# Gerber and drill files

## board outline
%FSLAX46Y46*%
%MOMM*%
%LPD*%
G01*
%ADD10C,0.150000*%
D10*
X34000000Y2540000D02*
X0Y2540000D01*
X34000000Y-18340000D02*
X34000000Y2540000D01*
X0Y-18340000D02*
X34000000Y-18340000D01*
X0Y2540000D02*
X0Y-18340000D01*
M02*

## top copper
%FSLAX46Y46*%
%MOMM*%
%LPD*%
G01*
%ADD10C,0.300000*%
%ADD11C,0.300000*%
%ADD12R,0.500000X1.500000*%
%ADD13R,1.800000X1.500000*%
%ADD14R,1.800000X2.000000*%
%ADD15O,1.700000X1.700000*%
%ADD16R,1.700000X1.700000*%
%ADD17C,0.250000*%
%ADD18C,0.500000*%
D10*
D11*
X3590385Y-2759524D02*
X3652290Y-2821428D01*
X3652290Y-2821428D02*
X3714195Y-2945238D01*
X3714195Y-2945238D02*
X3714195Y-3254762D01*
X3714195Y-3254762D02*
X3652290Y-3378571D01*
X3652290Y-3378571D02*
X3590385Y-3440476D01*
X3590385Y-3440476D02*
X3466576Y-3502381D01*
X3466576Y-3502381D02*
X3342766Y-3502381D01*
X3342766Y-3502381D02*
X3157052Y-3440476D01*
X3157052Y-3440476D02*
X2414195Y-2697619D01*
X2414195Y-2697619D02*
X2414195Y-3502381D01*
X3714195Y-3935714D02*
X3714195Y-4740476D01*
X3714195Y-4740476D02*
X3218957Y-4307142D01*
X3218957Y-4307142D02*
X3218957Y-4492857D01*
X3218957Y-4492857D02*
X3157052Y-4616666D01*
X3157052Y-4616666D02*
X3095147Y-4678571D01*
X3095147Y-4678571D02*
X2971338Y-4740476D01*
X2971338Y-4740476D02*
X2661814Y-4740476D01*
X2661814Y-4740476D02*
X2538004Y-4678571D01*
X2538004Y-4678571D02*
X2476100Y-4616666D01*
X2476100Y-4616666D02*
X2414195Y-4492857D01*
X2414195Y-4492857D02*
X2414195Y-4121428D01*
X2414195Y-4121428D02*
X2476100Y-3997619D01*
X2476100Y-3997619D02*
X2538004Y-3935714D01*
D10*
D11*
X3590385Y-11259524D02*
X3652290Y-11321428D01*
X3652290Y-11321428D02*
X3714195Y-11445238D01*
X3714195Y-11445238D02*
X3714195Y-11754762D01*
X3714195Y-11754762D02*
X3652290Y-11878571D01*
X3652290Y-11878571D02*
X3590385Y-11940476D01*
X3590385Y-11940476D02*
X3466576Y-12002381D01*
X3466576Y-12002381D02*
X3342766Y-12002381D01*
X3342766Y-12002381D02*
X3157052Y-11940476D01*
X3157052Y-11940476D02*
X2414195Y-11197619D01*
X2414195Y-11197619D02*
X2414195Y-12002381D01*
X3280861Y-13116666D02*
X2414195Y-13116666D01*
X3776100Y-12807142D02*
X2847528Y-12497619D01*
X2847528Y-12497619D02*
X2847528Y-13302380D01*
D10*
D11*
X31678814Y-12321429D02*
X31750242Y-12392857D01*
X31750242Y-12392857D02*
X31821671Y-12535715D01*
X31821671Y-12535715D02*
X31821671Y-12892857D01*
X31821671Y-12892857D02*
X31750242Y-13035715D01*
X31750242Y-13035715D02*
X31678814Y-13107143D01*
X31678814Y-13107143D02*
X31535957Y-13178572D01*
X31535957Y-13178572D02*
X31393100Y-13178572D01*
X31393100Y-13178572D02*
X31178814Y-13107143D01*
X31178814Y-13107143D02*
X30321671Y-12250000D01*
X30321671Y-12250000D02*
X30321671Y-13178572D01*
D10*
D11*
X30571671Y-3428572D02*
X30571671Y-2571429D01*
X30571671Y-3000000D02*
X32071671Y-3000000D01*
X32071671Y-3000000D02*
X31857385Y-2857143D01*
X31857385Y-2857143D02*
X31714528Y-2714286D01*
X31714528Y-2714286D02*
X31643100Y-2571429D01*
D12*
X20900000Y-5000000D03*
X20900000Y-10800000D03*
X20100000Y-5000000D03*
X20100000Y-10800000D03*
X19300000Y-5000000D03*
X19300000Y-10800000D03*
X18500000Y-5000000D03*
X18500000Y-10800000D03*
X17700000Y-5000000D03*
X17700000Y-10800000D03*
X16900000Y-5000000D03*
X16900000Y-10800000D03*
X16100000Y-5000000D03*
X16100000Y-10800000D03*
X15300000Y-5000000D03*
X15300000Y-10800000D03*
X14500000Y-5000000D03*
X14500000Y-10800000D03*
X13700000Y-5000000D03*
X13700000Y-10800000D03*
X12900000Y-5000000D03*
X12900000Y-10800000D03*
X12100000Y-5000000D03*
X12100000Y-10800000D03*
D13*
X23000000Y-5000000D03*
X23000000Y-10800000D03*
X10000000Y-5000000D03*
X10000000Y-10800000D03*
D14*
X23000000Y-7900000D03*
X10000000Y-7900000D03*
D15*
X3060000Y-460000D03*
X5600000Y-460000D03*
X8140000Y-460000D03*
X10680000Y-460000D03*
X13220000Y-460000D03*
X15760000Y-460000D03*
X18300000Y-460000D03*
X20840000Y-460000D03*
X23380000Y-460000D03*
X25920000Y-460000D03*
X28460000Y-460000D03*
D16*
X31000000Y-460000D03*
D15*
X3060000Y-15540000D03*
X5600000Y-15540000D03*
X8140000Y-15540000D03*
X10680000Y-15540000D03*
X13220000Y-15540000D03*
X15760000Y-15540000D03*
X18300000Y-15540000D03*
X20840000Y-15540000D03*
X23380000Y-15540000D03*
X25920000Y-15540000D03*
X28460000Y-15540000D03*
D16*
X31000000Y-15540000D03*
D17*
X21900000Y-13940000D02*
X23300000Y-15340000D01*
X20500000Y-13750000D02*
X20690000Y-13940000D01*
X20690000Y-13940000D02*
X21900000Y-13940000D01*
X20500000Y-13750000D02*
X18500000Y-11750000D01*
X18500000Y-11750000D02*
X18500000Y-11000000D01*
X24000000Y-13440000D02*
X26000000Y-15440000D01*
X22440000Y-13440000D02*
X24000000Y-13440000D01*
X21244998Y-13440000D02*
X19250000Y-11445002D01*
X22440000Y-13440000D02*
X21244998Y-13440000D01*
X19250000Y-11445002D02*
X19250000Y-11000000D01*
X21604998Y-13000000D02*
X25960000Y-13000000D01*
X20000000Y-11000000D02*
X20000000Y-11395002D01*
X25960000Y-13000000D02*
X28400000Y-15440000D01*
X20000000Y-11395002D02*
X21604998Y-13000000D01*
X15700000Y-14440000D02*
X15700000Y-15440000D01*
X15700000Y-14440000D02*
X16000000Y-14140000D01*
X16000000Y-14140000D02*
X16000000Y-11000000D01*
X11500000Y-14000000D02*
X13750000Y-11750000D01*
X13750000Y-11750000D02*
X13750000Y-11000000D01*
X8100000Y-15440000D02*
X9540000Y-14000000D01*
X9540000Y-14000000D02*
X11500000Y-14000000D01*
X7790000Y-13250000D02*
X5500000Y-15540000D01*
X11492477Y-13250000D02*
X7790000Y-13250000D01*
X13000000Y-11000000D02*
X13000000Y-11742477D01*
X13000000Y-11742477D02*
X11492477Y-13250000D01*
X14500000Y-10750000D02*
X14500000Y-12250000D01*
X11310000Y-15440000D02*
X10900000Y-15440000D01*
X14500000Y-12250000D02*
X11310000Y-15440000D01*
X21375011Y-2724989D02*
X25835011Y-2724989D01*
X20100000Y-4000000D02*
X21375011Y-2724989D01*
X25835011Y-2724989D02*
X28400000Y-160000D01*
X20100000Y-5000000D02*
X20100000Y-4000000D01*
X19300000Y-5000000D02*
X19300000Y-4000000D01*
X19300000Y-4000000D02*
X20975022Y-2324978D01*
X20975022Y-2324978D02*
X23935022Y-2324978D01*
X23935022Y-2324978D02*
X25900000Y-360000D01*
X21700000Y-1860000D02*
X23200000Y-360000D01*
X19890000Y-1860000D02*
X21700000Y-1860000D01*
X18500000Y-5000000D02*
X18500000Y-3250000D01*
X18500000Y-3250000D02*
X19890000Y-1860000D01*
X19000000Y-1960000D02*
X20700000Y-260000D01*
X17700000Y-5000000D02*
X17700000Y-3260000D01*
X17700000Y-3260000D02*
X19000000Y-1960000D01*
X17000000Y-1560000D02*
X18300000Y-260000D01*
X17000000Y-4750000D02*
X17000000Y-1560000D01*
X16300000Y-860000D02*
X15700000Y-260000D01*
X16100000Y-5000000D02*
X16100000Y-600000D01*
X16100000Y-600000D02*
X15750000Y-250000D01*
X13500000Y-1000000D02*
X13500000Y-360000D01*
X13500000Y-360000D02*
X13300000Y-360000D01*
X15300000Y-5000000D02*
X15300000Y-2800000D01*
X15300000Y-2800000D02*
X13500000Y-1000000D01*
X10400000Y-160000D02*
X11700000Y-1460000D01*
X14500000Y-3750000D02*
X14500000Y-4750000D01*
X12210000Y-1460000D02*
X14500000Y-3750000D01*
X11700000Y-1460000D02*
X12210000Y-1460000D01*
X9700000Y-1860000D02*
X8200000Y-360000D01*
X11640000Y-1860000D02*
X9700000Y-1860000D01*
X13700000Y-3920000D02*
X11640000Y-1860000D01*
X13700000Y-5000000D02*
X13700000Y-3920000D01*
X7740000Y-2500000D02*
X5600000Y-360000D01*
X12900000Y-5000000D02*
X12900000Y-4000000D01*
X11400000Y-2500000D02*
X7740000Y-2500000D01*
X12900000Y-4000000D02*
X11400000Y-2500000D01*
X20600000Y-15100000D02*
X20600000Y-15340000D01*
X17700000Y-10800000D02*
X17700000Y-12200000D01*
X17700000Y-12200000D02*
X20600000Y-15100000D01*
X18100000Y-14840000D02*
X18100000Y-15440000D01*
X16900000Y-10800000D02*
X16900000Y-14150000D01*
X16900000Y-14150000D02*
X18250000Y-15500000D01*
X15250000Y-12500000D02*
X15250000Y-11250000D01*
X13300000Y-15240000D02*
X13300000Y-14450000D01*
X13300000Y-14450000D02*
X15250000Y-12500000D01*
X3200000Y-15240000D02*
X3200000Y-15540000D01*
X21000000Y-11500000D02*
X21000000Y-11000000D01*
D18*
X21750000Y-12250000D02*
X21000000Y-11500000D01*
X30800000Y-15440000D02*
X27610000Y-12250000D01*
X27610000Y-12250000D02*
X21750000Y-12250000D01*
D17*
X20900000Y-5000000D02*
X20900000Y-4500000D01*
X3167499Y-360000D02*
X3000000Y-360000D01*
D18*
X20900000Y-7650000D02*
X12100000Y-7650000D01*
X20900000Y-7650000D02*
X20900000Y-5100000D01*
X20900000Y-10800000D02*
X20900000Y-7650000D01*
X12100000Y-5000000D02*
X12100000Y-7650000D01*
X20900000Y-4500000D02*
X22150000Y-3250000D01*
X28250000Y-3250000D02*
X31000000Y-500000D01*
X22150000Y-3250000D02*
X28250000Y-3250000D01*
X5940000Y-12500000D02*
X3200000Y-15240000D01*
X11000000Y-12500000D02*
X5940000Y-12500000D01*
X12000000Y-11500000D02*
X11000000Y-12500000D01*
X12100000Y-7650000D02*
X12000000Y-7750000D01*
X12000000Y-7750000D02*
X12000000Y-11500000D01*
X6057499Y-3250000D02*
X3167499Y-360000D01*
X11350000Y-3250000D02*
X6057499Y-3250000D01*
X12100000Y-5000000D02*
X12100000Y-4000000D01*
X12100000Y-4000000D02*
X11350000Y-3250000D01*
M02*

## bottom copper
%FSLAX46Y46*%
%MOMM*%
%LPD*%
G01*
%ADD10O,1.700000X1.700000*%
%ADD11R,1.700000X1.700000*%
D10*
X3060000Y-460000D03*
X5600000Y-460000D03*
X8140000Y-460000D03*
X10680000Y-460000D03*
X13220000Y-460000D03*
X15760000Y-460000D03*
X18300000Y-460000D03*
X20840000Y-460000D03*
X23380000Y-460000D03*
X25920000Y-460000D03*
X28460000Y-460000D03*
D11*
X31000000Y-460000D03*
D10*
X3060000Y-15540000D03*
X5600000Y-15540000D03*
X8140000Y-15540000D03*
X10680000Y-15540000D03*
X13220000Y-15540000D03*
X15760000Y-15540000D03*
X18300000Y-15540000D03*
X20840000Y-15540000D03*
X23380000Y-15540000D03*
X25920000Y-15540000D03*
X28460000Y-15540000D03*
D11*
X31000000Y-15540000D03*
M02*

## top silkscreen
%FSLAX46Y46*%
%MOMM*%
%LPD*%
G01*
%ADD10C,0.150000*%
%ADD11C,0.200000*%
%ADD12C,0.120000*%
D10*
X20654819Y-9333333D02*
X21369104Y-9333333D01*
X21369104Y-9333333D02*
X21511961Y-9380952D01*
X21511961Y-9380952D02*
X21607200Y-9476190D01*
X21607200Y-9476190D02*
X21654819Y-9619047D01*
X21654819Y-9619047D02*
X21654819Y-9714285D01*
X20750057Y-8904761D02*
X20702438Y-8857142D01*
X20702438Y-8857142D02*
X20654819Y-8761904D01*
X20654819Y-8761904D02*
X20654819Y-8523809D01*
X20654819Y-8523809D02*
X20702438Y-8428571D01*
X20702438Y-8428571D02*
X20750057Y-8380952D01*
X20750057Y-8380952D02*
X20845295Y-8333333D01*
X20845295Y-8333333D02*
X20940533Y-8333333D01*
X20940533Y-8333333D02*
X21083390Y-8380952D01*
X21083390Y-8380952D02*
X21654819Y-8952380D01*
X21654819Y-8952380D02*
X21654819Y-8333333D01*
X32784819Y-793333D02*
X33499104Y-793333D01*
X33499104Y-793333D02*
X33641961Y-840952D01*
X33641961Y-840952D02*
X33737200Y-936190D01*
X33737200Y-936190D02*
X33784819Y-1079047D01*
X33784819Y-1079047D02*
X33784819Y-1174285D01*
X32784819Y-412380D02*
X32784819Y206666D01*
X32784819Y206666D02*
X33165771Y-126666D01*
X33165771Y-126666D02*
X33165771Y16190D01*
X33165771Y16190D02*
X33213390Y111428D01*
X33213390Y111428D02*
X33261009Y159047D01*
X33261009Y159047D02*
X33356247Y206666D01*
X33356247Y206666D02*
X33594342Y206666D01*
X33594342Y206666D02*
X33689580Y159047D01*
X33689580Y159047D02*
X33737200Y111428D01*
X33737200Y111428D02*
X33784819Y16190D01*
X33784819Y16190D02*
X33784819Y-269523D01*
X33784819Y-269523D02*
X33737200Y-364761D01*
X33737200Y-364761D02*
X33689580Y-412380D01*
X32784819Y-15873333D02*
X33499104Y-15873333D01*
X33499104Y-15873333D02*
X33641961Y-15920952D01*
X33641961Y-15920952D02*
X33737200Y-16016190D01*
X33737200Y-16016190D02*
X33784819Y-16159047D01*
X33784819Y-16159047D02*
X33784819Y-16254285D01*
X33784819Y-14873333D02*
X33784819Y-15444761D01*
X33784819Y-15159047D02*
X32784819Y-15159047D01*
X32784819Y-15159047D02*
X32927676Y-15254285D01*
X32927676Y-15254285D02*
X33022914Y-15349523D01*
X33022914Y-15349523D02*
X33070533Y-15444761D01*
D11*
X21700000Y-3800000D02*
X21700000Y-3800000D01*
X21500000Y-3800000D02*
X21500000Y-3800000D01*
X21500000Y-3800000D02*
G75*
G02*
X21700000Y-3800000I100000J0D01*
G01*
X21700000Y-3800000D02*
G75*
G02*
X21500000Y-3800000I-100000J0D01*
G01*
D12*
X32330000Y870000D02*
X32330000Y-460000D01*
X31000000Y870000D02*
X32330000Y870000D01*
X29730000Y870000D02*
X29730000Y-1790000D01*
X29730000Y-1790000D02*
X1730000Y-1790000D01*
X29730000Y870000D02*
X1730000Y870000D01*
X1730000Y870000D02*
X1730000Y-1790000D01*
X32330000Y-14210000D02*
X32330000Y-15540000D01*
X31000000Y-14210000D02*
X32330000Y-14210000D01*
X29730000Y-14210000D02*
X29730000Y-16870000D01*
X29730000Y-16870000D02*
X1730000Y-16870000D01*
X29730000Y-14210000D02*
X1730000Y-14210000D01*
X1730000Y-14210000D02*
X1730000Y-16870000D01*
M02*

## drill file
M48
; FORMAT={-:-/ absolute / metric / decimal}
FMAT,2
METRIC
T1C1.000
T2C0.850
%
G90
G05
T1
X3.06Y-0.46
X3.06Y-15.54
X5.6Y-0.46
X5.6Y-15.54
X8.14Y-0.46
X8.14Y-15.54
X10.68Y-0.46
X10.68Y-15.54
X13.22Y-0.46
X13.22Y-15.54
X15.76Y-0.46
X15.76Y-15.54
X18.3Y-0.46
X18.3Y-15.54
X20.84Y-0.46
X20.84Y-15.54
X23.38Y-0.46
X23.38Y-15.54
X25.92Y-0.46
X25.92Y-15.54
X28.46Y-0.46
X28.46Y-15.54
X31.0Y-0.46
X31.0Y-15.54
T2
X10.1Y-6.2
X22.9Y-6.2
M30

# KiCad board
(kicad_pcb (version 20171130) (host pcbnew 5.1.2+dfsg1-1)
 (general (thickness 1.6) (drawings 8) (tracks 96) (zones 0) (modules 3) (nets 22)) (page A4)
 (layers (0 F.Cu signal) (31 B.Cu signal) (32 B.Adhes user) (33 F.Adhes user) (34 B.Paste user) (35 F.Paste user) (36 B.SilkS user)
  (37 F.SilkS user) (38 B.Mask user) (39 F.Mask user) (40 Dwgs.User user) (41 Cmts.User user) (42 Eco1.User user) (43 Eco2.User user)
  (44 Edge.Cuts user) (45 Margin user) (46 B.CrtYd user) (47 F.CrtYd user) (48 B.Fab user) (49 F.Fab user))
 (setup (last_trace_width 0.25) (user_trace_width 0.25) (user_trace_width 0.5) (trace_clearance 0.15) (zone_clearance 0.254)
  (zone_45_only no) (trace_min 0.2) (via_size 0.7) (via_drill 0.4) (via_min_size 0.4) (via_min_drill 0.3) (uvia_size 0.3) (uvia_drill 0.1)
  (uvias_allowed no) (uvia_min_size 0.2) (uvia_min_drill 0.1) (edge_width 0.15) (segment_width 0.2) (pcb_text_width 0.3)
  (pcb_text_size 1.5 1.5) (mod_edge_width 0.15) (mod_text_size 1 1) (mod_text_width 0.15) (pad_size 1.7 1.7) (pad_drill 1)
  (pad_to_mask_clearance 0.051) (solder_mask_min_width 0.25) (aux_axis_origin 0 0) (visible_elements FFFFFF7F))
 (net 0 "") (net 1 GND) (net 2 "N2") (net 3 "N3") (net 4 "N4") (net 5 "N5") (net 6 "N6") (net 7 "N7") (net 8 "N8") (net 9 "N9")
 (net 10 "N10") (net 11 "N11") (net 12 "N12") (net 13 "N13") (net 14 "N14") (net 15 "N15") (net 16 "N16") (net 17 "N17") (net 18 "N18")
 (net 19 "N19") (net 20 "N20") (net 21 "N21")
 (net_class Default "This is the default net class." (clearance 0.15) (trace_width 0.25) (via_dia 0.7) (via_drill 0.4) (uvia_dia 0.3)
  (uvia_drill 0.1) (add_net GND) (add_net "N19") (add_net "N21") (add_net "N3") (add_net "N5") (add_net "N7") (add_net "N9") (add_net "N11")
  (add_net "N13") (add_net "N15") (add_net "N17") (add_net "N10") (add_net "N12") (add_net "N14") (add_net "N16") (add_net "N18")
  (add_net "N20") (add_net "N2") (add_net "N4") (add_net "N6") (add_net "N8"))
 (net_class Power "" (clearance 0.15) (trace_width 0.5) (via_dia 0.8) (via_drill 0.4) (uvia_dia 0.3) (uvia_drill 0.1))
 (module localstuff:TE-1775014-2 (layer F.Cu) (at 16.5 7.9 180)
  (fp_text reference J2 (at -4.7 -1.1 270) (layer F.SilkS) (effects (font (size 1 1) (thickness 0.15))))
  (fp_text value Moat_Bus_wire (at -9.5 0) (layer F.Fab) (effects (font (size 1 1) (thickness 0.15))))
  (fp_line (start -5.2 4.1) (end -5.2 4.1) (layer F.SilkS) (width 0.2))
  (fp_line (start -5 4.1) (end -5 4.1) (layer F.SilkS) (width 0.2))
  (fp_arc (start -5.1 4.1) (end -5.2 4.1) (angle -180) (layer F.SilkS) (width 0.2))
  (fp_arc (start -5.1 4.1) (end -5 4.1) (angle -180) (layer F.SilkS) (width 0.2))
  (pad 1 smd rect (at -4.4 2.9 180) (size 0.5 1.5) (layers F.Cu F.Paste) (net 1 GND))
  (pad 2 smd rect (at -4.4 -2.9 180) (size 0.5 1.5) (layers F.Cu F.Paste) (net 1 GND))
  (pad 3 smd rect (at -3.6 2.9 180) (size 0.5 1.5) (layers F.Cu F.Paste) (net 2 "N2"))
  (pad 4 smd rect (at -3.6 -2.9 180) (size 0.5 1.5) (layers F.Cu F.Paste) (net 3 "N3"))
  (pad 5 smd rect (at -2.8 2.9 180) (size 0.5 1.5) (layers F.Cu F.Paste) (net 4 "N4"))
  (pad 6 smd rect (at -2.8 -2.9 180) (size 0.5 1.5) (layers F.Cu F.Paste) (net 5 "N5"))
  (pad 7 smd rect (at -2 2.9 180) (size 0.5 1.5) (layers F.Cu F.Paste) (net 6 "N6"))
  (pad 8 smd rect (at -2 -2.9 180) (size 0.5 1.5) (layers F.Cu F.Paste) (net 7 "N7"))
  (pad 9 smd rect (at -1.2 2.9 180) (size 0.5 1.5) (layers F.Cu F.Paste) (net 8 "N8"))
  (pad 10 smd rect (at -1.2 -2.9 180) (size 0.5 1.5) (layers F.Cu F.Paste) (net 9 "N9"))
  (pad 11 smd rect (at -0.4 2.9 180) (size 0.5 1.5) (layers F.Cu F.Paste) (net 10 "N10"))
  (pad 12 smd rect (at -0.4 -2.9 180) (size 0.5 1.5) (layers F.Cu F.Paste) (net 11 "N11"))
  (pad 13 smd rect (at 0.4 2.9 180) (size 0.5 1.5) (layers F.Cu F.Paste) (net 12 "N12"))
  (pad 14 smd rect (at 0.4 -2.9 180) (size 0.5 1.5) (layers F.Cu F.Paste) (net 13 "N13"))
  (pad 15 smd rect (at 1.2 2.9 180) (size 0.5 1.5) (layers F.Cu F.Paste) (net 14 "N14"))
  (pad 16 smd rect (at 1.2 -2.9 180) (size 0.5 1.5) (layers F.Cu F.Paste) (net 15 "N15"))
  (pad 17 smd rect (at 2 2.9 180) (size 0.5 1.5) (layers F.Cu F.Paste) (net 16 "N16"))
  (pad 18 smd rect (at 2 -2.9 180) (size 0.5 1.5) (layers F.Cu F.Paste) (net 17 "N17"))
  (pad 19 smd rect (at 2.8 2.9 180) (size 0.5 1.5) (layers F.Cu F.Paste) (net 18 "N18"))
  (pad 20 smd rect (at 2.8 -2.9 180) (size 0.5 1.5) (layers F.Cu F.Paste) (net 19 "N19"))
  (pad 21 smd rect (at 3.6 2.9 180) (size 0.5 1.5) (layers F.Cu F.Paste) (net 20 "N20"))
  (pad 22 smd rect (at 3.6 -2.9 180) (size 0.5 1.5) (layers F.Cu F.Paste) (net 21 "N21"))
  (pad 23 smd rect (at 4.4 2.9 180) (size 0.5 1.5) (layers F.Cu F.Paste) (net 1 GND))
  (pad 24 smd rect (at 4.4 -2.9 180) (size 0.5 1.5) (layers F.Cu F.Paste) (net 1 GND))
  (pad MNT smd rect (at -6.5 2.9 270) (size 1.5 1.8) (layers F.Cu F.Paste))
  (pad MNT smd rect (at -6.5 -2.9 270) (size 1.5 1.8) (layers F.Cu F.Paste))
  (pad MNT smd rect (at 6.5 2.9 270) (size 1.5 1.8) (layers F.Cu F.Paste))
  (pad MNT smd rect (at 6.5 -2.9 270) (size 1.5 1.8) (layers F.Cu F.Paste))
  (pad MNT smd rect (at -6.5 0 180) (size 1.8 2) (layers F.Cu F.Paste))
  (pad MNT smd rect (at 6.5 0 180) (size 1.8 2) (layers F.Cu F.Paste))
  (pad 31 np_thru_hole circle (at -6.4 1.7 180) (size 0.85 0) (drill 0.85) (layers *.Cu *.Mask))
  (pad 32 np_thru_hole circle (at 6.4 1.7 180) (size 0.85 0) (drill 0.85) (layers *.Cu *.Mask)))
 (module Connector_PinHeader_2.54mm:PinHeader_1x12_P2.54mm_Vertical (layer F.Cu) (at 31 0.46 270)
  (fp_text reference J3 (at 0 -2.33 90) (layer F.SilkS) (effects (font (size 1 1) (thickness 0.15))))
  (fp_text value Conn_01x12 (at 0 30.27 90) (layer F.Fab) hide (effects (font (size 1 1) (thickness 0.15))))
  (fp_line (start -1.33 -1.33) (end 0 -1.33) (layer F.SilkS) (width 0.12))
  (fp_line (start -1.33 0) (end -1.33 -1.33) (layer F.SilkS) (width 0.12))
  (fp_line (start -1.33 1.27) (end 1.33 1.27) (layer F.SilkS) (width 0.12))
  (fp_line (start 1.33 1.27) (end 1.33 29.27) (layer F.SilkS) (width 0.12))
  (fp_line (start -1.33 1.27) (end -1.33 29.27) (layer F.SilkS) (width 0.12))
  (fp_line (start -1.33 29.27) (end 1.33 29.27) (layer F.SilkS) (width 0.12))
  (pad 12 thru_hole oval (at 0 27.94 270) (size 1.7 1.7) (drill 1) (layers *.Cu *.Mask) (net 1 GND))
  (pad 11 thru_hole oval (at 0 25.4 270) (size 1.7 1.7) (drill 1) (layers *.Cu *.Mask) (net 20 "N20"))
  (pad 10 thru_hole oval (at 0 22.86 270) (size 1.7 1.7) (drill 1) (layers *.Cu *.Mask) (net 18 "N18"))
  (pad 9 thru_hole oval (at 0 20.32 270) (size 1.7 1.7) (drill 1) (layers *.Cu *.Mask) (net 16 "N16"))
  (pad 8 thru_hole oval (at 0 17.78 270) (size 1.7 1.7) (drill 1) (layers *.Cu *.Mask) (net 14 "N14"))
  (pad 7 thru_hole oval (at 0 15.24 270) (size 1.7 1.7) (drill 1) (layers *.Cu *.Mask) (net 12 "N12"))
  (pad 6 thru_hole oval (at 0 12.7 270) (size 1.7 1.7) (drill 1) (layers *.Cu *.Mask) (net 10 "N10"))
  (pad 5 thru_hole oval (at 0 10.16 270) (size 1.7 1.7) (drill 1) (layers *.Cu *.Mask) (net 8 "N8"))
  (pad 4 thru_hole oval (at 0 7.62 270) (size 1.7 1.7) (drill 1) (layers *.Cu *.Mask) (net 6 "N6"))
  (pad 3 thru_hole oval (at 0 5.08 270) (size 1.7 1.7) (drill 1) (layers *.Cu *.Mask) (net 4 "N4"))
  (pad 2 thru_hole oval (at 0 2.54 270) (size 1.7 1.7) (drill 1) (layers *.Cu *.Mask) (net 2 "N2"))
  (pad 1 thru_hole rect (at 0 0 270) (size 1.7 1.7) (drill 1) (layers *.Cu *.Mask) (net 1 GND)))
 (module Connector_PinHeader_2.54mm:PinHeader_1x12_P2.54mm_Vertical (layer F.Cu) (at 31 15.54 270)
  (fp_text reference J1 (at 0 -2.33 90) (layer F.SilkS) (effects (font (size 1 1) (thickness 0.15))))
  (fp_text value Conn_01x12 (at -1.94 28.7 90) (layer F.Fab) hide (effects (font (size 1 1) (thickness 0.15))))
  (fp_line (start -1.33 -1.33) (end 0 -1.33) (layer F.SilkS) (width 0.12))
  (fp_line (start -1.33 0) (end -1.33 -1.33) (layer F.SilkS) (width 0.12))
  (fp_line (start -1.33 1.27) (end 1.33 1.27) (layer F.SilkS) (width 0.12))
  (fp_line (start 1.33 1.27) (end 1.33 29.27) (layer F.SilkS) (width 0.12))
  (fp_line (start -1.33 1.27) (end -1.33 29.27) (layer F.SilkS) (width 0.12))
  (fp_line (start -1.33 29.27) (end 1.33 29.27) (layer F.SilkS) (width 0.12))
  (pad 12 thru_hole oval (at 0 27.94 270) (size 1.7 1.7) (drill 1) (layers *.Cu *.Mask) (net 1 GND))
  (pad 11 thru_hole oval (at 0 25.4 270) (size 1.7 1.7) (drill 1) (layers *.Cu *.Mask) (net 21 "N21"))
  (pad 10 thru_hole oval (at 0 22.86 270) (size 1.7 1.7) (drill 1) (layers *.Cu *.Mask) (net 19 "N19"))
  (pad 9 thru_hole oval (at 0 20.32 270) (size 1.7 1.7) (drill 1) (layers *.Cu *.Mask) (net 17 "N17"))
  (pad 8 thru_hole oval (at 0 17.78 270) (size 1.7 1.7) (drill 1) (layers *.Cu *.Mask) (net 15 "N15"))
  (pad 7 thru_hole oval (at 0 15.24 270) (size 1.7 1.7) (drill 1) (layers *.Cu *.Mask) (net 13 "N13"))
  (pad 6 thru_hole oval (at 0 12.7 270) (size 1.7 1.7) (drill 1) (layers *.Cu *.Mask) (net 11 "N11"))
  (pad 5 thru_hole oval (at 0 10.16 270) (size 1.7 1.7) (drill 1) (layers *.Cu *.Mask) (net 9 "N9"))
  (pad 4 thru_hole oval (at 0 7.62 270) (size 1.7 1.7) (drill 1) (layers *.Cu *.Mask) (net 7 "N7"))
  (pad 3 thru_hole oval (at 0 5.08 270) (size 1.7 1.7) (drill 1) (layers *.Cu *.Mask) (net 5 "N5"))
  (pad 2 thru_hole oval (at 0 2.54 270) (size 1.7 1.7) (drill 1) (layers *.Cu *.Mask) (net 3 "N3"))
  (pad 1 thru_hole rect (at 0 0 270) (size 1.7 1.7) (drill 1) (layers *.Cu *.Mask) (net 1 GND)))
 (gr_line (start 34 -2.54) (end 0 -2.54) (layer Edge.Cuts) (width 0.15))
 (gr_line (start 34 18.34) (end 34 -2.54) (layer Edge.Cuts) (width 0.15))
 (gr_line (start 0 18.34) (end 34 18.34) (layer Edge.Cuts) (width 0.15))
 (gr_line (start 0 -2.54) (end 0 18.34) (layer Edge.Cuts) (width 0.15))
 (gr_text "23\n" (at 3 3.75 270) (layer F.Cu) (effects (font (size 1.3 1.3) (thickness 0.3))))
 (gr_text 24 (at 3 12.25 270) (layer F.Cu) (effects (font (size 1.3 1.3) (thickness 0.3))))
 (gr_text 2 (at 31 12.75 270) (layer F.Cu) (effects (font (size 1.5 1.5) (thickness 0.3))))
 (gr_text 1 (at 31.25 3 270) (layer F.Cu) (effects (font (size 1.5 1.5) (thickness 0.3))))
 (segment (start 21.9 13.94) (end 23.3 15.34) (width 0.25) (layer F.Cu) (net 7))
 (segment (start 20.5 13.75) (end 20.69 13.94) (width 0.25) (layer F.Cu) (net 7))
 (segment (start 20.69 13.94) (end 21.9 13.94) (width 0.25) (layer F.Cu) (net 7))
 (segment (start 20.5 13.75) (end 18.5 11.75) (width 0.25) (layer F.Cu) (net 7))
 (segment (start 18.5 11.75) (end 18.5 11) (width 0.25) (layer F.Cu) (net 7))
 (segment (start 24 13.44) (end 26 15.44) (width 0.25) (layer F.Cu) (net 5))
 (segment (start 22.44 13.44) (end 24 13.44) (width 0.25) (layer F.Cu) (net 5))
 (segment (start 21.244998 13.44) (end 19.25 11.445002) (width 0.25) (layer F.Cu) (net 5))
 (segment (start 22.44 13.44) (end 21.244998 13.44) (width 0.25) (layer F.Cu) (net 5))
 (segment (start 19.25 11.445002) (end 19.25 11) (width 0.25) (layer F.Cu) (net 5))
 (segment (start 21.604998 13) (end 25.96 13) (width 0.25) (layer F.Cu) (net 3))
 (segment (start 20 11) (end 20 11.395002) (width 0.25) (layer F.Cu) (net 3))
 (segment (start 25.96 13) (end 28.4 15.44) (width 0.25) (layer F.Cu) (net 3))
 (segment (start 20 11.395002) (end 21.604998 13) (width 0.25) (layer F.Cu) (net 3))
 (segment (start 15.7 14.44) (end 15.7 15.44) (width 0.25) (layer F.Cu) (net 13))
 (segment (start 15.7 14.44) (end 16 14.14) (width 0.25) (layer F.Cu) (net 13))
 (segment (start 16 14.14) (end 16 11) (width 0.25) (layer F.Cu) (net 13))
 (segment (start 11.5 14) (end 13.75 11.75) (width 0.25) (layer F.Cu) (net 19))
 (segment (start 13.75 11.75) (end 13.75 11) (width 0.25) (layer F.Cu) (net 19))
 (segment (start 8.1 15.44) (end 9.54 14) (width 0.25) (layer F.Cu) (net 19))
 (segment (start 9.54 14) (end 11.5 14) (width 0.25) (layer F.Cu) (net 19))
 (segment (start 7.79 13.25) (end 5.5 15.54) (width 0.25) (layer F.Cu) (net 21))
 (segment (start 11.492477 13.25) (end 7.79 13.25) (width 0.25) (layer F.Cu) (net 21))
 (segment (start 13 11) (end 13 11.742477) (width 0.25) (layer F.Cu) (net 21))
 (segment (start 13 11.742477) (end 11.492477 13.25) (width 0.25) (layer F.Cu) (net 21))
 (segment (start 14.5 10.75) (end 14.5 12.25) (width 0.25) (layer F.Cu) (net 17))
 (segment (start 11.31 15.44) (end 10.9 15.44) (width 0.25) (layer F.Cu) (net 17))
 (segment (start 14.5 12.25) (end 11.31 15.44) (width 0.25) (layer F.Cu) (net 17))
 (segment (start 21.375011 2.724989) (end 25.835011 2.724989) (width 0.25) (layer F.Cu) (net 2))
 (segment (start 20.1 4) (end 21.375011 2.724989) (width 0.25) (layer F.Cu) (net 2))
 (segment (start 25.835011 2.724989) (end 28.4 0.16) (width 0.25) (layer F.Cu) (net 2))
 (segment (start 20.1 5) (end 20.1 4) (width 0.25) (layer F.Cu) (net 2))
 (segment (start 19.3 5) (end 19.3 4) (width 0.25) (layer F.Cu) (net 4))
 (segment (start 19.3 4) (end 20.975022 2.324978) (width 0.25) (layer F.Cu) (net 4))
 (segment (start 20.975022 2.324978) (end 23.935022 2.324978) (width 0.25) (layer F.Cu) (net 4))
 (segment (start 23.935022 2.324978) (end 25.9 0.36) (width 0.25) (layer F.Cu) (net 4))
 (segment (start 21.7 1.86) (end 23.2 0.36) (width 0.25) (layer F.Cu) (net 6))
 (segment (start 19.89 1.86) (end 21.7 1.86) (width 0.25) (layer F.Cu) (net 6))
 (segment (start 18.5 5) (end 18.5 3.25) (width 0.25) (layer F.Cu) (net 6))
 (segment (start 18.5 3.25) (end 19.89 1.86) (width 0.25) (layer F.Cu) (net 6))
 (segment (start 19 1.96) (end 20.7 0.26) (width 0.25) (layer F.Cu) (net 8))
 (segment (start 17.7 5) (end 17.7 3.26) (width 0.25) (layer F.Cu) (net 8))
 (segment (start 17.7 3.26) (end 19 1.96) (width 0.25) (layer F.Cu) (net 8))
 (segment (start 17 1.56) (end 18.3 0.26) (width 0.25) (layer F.Cu) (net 10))
 (segment (start 17 4.75) (end 17 1.56) (width 0.25) (layer F.Cu) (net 10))
 (segment (start 16.3 0.86) (end 15.7 0.26) (width 0.25) (layer F.Cu) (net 12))
 (segment (start 16.1 5) (end 16.1 0.6) (width 0.25) (layer F.Cu) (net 12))
 (segment (start 16.1 0.6) (end 15.75 0.25) (width 0.25) (layer F.Cu) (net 12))
 (segment (start 13.5 1) (end 13.5 0.36) (width 0.25) (layer F.Cu) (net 14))
 (segment (start 13.5 0.36) (end 13.3 0.36) (width 0.25) (layer F.Cu) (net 14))
 (segment (start 15.3 5) (end 15.3 2.8) (width 0.25) (layer F.Cu) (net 14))
 (segment (start 15.3 2.8) (end 13.5 1) (width 0.25) (layer F.Cu) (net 14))
 (segment (start 10.4 0.16) (end 11.7 1.46) (width 0.25) (layer F.Cu) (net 16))
 (segment (start 14.5 3.75) (end 14.5 4.75) (width 0.25) (layer F.Cu) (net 16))
 (segment (start 12.21 1.46) (end 14.5 3.75) (width 0.25) (layer F.Cu) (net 16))
 (segment (start 11.7 1.46) (end 12.21 1.46) (width 0.25) (layer F.Cu) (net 16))
 (segment (start 9.7 1.86) (end 8.2 0.36) (width 0.25) (layer F.Cu) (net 18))
 (segment (start 11.64 1.86) (end 9.7 1.86) (width 0.25) (layer F.Cu) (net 18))
 (segment (start 13.7 3.92) (end 11.64 1.86) (width 0.25) (layer F.Cu) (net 18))
 (segment (start 13.7 5) (end 13.7 3.92) (width 0.25) (layer F.Cu) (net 18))
 (segment (start 7.74 2.5) (end 5.6 0.36) (width 0.25) (layer F.Cu) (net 20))
 (segment (start 12.9 5) (end 12.9 4) (width 0.25) (layer F.Cu) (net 20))
 (segment (start 11.4 2.5) (end 7.74 2.5) (width 0.25) (layer F.Cu) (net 20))
 (segment (start 12.9 4) (end 11.4 2.5) (width 0.25) (layer F.Cu) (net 20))
 (segment (start 20.6 15.1) (end 20.6 15.34) (width 0.25) (layer F.Cu) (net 9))
 (segment (start 17.7 10.8) (end 17.7 12.2) (width 0.25) (layer F.Cu) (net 9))
 (segment (start 17.7 12.2) (end 20.6 15.1) (width 0.25) (layer F.Cu) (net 9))
 (segment (start 18.1 14.84) (end 18.1 15.44) (width 0.25) (layer F.Cu) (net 11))
 (segment (start 16.9 10.8) (end 16.9 14.15) (width 0.25) (layer F.Cu) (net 11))
 (segment (start 16.9 14.15) (end 18.25 15.5) (width 0.25) (layer F.Cu) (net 11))
 (segment (start 15.25 12.5) (end 15.25 11.25) (width 0.25) (layer F.Cu) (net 15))
 (segment (start 13.3 15.24) (end 13.3 14.45) (width 0.25) (layer F.Cu) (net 15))
 (segment (start 13.3 14.45) (end 15.25 12.5) (width 0.25) (layer F.Cu) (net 15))
 (segment (start 3.2 15.24) (end 3.2 15.54) (width 0.25) (layer F.Cu) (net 1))
 (segment (start 21 11.5) (end 21 11) (width 0.25) (layer F.Cu) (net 1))
 (segment (start 21.75 12.25) (end 21 11.5) (width 0.5) (layer F.Cu) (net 1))
 (segment (start 30.8 15.44) (end 27.61 12.25) (width 0.5) (layer F.Cu) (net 1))
 (segment (start 27.61 12.25) (end 21.75 12.25) (width 0.5) (layer F.Cu) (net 1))
 (segment (start 20.9 5) (end 20.9 4.5) (width 0.25) (layer F.Cu) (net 1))
 (segment (start 3.167499 0.36) (end 3 0.36) (width 0.25) (layer F.Cu) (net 1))
 (segment (start 20.9 7.65) (end 12.1 7.65) (width 0.5) (layer F.Cu) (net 1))
 (segment (start 20.9 7.65) (end 20.9 5.1) (width 0.5) (layer F.Cu) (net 1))
 (segment (start 20.9 10.8) (end 20.9 7.65) (width 0.5) (layer F.Cu) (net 1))
 (segment (start 12.1 5) (end 12.1 7.65) (width 0.5) (layer F.Cu) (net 1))
 (segment (start 20.9 4.5) (end 22.15 3.25) (width 0.5) (layer F.Cu) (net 1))
 (segment (start 28.25 3.25) (end 31 0.5) (width 0.5) (layer F.Cu) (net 1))
 (segment (start 22.15 3.25) (end 28.25 3.25) (width 0.5) (layer F.Cu) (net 1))
 (segment (start 5.94 12.5) (end 3.2 15.24) (width 0.5) (layer F.Cu) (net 1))
 (segment (start 11 12.5) (end 5.94 12.5) (width 0.5) (layer F.Cu) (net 1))
 (segment (start 12 11.5) (end 11 12.5) (width 0.5) (layer F.Cu) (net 1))
 (segment (start 12.1 7.65) (end 12 7.75) (width 0.5) (layer F.Cu) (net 1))
 (segment (start 12 7.75) (end 12 11.5) (width 0.5) (layer F.Cu) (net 1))
 (segment (start 6.057499 3.25) (end 3.167499 0.36) (width 0.5) (layer F.Cu) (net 1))
 (segment (start 11.35 3.25) (end 6.057499 3.25) (width 0.5) (layer F.Cu) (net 1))
 (segment (start 12.1 5) (end 12.1 4) (width 0.5) (layer F.Cu) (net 1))
 (segment (start 12.1 4) (end 11.35 3.25) (width 0.5) (layer F.Cu) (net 1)))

